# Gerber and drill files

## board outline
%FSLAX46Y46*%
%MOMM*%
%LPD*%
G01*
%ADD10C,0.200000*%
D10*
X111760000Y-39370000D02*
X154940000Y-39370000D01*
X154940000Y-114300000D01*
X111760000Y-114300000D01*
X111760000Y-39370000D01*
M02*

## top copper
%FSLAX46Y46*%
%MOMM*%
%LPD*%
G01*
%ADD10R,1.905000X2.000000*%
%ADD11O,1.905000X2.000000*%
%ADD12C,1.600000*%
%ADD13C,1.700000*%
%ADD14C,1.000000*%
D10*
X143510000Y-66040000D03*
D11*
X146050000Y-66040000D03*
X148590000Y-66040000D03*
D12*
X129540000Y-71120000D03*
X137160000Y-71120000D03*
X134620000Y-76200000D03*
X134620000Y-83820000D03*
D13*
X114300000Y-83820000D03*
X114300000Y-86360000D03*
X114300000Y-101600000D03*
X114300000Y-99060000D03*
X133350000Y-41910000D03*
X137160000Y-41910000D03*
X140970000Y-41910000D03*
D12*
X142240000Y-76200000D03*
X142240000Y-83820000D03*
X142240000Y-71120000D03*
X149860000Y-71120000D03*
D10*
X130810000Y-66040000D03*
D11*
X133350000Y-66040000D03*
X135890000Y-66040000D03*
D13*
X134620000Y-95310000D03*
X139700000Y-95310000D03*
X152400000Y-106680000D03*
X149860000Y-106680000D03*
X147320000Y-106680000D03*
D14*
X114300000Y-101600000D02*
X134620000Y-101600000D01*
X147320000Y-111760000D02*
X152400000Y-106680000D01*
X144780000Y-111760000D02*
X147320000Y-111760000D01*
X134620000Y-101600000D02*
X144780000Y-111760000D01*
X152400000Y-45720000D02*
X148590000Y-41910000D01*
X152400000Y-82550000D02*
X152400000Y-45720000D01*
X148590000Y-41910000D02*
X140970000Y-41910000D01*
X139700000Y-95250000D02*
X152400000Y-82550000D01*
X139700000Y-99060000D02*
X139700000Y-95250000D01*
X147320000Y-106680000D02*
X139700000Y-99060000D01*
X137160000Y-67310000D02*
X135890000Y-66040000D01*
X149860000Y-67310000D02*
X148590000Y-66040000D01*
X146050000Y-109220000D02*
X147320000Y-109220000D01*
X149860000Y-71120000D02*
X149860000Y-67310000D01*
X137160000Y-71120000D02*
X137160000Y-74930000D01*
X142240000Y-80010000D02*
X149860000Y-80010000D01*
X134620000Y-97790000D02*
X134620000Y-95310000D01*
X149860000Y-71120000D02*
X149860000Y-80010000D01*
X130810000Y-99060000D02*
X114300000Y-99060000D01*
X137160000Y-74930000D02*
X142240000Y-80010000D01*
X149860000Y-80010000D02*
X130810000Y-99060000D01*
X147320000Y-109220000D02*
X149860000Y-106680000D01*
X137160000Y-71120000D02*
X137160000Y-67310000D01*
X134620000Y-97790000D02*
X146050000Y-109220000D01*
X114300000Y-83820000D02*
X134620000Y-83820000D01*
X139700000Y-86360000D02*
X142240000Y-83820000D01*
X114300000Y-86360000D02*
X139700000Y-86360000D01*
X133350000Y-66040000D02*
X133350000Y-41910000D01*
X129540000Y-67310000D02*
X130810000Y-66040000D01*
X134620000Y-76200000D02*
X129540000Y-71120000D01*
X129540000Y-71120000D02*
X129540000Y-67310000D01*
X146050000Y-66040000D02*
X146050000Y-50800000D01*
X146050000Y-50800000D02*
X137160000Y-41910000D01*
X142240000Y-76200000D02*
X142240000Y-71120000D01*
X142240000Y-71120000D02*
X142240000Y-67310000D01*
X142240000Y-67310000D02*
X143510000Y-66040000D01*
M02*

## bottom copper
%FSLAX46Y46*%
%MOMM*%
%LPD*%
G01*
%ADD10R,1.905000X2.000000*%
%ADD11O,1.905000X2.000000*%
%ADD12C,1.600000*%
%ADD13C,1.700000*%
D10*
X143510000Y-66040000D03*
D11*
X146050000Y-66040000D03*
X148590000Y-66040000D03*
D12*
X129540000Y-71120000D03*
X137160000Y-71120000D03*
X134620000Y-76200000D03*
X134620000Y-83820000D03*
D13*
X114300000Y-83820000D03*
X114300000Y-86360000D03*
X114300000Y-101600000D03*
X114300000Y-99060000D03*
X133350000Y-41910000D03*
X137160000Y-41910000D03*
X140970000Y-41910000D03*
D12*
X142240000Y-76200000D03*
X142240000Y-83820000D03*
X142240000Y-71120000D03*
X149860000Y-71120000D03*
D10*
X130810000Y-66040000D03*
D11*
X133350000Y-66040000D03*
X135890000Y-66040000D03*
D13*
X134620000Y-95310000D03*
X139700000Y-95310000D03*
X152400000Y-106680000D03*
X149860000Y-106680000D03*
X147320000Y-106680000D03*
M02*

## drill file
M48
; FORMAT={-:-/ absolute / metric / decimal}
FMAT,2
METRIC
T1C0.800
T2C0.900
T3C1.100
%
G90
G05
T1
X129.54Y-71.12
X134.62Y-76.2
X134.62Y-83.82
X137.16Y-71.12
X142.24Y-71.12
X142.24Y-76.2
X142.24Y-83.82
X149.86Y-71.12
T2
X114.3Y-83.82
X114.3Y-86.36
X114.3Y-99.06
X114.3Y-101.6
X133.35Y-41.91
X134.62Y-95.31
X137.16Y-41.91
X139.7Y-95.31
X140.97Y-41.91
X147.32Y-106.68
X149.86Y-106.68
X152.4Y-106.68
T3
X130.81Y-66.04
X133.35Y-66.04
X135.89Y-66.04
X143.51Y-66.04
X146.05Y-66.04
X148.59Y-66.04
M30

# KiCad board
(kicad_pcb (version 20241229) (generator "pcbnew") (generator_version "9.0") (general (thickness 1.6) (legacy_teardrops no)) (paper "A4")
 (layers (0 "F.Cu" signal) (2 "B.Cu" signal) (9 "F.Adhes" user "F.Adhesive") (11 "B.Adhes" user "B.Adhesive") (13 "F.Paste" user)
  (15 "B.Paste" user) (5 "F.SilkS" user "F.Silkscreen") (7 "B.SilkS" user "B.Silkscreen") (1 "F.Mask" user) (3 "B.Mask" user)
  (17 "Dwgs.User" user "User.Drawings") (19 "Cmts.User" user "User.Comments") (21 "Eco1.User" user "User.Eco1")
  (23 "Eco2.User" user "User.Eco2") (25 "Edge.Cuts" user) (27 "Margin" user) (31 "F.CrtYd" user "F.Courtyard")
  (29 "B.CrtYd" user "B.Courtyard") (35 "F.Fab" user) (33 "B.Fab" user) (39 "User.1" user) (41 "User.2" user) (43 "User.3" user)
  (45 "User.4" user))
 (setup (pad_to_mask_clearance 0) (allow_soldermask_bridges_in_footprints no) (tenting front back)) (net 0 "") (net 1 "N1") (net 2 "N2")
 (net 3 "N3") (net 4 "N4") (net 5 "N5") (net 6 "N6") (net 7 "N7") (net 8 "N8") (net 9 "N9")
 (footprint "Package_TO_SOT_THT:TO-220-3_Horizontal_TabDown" (layer "F.Cu") (at 143.51 66.04)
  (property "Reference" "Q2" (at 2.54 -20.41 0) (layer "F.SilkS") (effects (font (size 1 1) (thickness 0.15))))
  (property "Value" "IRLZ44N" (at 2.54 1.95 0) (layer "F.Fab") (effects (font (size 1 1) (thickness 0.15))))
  (pad "1" thru_hole rect (at 0 0) (size 1.905 2) (drill 1.1) (layers "*.Cu" "*.Mask") (remove_unused_layers no) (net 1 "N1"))
  (pad "2" thru_hole oval (at 2.54 0) (size 1.905 2) (drill 1.1) (layers "*.Cu" "*.Mask") (remove_unused_layers no) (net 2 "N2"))
  (pad "3" thru_hole oval (at 5.08 0) (size 1.905 2) (drill 1.1) (layers "*.Cu" "*.Mask") (remove_unused_layers no) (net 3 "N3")))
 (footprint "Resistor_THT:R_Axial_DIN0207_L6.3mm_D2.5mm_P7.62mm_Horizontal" (layer "F.Cu") (at 129.54 71.12)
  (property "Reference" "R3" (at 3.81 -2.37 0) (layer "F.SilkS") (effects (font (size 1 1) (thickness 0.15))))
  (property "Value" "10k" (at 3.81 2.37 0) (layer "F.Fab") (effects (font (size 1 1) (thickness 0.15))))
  (pad "1" thru_hole circle (at 0 0) (size 1.6 1.6) (drill 0.8) (layers "*.Cu" "*.Mask") (remove_unused_layers no) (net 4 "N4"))
  (pad "2" thru_hole circle (at 7.62 0) (size 1.6 1.6) (drill 0.8) (layers "*.Cu" "*.Mask") (remove_unused_layers no) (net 3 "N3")))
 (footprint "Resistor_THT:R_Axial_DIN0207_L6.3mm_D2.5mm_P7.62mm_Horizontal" (layer "F.Cu") (at 134.62 76.2 -90)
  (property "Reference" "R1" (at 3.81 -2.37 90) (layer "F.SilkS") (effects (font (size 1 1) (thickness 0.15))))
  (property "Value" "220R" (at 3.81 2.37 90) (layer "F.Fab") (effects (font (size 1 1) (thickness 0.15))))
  (pad "1" thru_hole circle (at 0 0 270) (size 1.6 1.6) (drill 0.8) (layers "*.Cu" "*.Mask") (remove_unused_layers no) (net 4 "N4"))
  (pad "2" thru_hole circle (at 7.62 0 270) (size 1.6 1.6) (drill 0.8) (layers "*.Cu" "*.Mask") (remove_unused_layers no) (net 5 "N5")))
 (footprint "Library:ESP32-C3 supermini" (layer "F.Cu") (at 121.92 91.44)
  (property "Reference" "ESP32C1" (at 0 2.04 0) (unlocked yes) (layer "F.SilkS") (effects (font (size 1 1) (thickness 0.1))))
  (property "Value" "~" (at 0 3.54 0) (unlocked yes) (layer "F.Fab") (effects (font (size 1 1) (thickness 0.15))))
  (pad "0" thru_hole circle (at -7.62 -7.62) (size 1.7 1.7) (drill 0.9) (layers "*.Cu" "*.Mask") (remove_unused_layers yes)
   (keep_end_layers yes) (zone_layer_connections) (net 5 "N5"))
  (pad "1" thru_hole circle (at -7.62 -5.08) (size 1.7 1.7) (drill 0.9) (layers "*.Cu" "*.Mask") (remove_unused_layers yes)
   (keep_end_layers yes) (zone_layer_connections) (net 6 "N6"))
  (pad "5V" thru_hole circle (at -7.62 10.16) (size 1.7 1.7) (drill 0.9) (layers "*.Cu" "*.Mask") (remove_unused_layers yes)
   (keep_end_layers yes) (zone_layer_connections) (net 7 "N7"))
  (pad "GND" thru_hole circle (at -7.62 7.62) (size 1.7 1.7) (drill 0.9) (layers "*.Cu" "*.Mask") (remove_unused_layers yes)
   (keep_end_layers yes) (zone_layer_connections) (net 3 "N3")))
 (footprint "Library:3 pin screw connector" (layer "F.Cu") (at 137.16 41.91)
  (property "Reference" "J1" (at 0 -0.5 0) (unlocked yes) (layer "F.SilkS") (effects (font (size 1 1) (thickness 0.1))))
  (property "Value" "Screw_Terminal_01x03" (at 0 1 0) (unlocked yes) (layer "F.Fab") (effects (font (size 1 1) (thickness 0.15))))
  (pad "1" thru_hole circle (at -3.81 0) (size 1.7 1.7) (drill 0.9) (layers "*.Cu" "*.Mask") (remove_unused_layers yes)
   (keep_end_layers yes) (zone_layer_connections) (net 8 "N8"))
  (pad "2" thru_hole circle (at 0 0) (size 1.7 1.7) (drill 0.9) (layers "*.Cu" "*.Mask") (remove_unused_layers yes) (keep_end_layers yes)
   (zone_layer_connections) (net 2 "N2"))
  (pad "3" thru_hole circle (at 3.81 0) (size 1.7 1.7) (drill 0.9) (layers "*.Cu" "*.Mask") (remove_unused_layers yes) (keep_end_layers yes)
   (zone_layer_connections) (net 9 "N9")))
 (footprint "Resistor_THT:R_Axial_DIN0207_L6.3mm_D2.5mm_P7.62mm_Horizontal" (layer "F.Cu") (at 142.24 76.2 -90)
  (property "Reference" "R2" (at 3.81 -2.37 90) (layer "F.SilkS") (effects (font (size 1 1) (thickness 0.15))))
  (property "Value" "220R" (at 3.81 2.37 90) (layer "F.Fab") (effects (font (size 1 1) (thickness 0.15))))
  (pad "1" thru_hole circle (at 0 0 270) (size 1.6 1.6) (drill 0.8) (layers "*.Cu" "*.Mask") (remove_unused_layers no) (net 1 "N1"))
  (pad "2" thru_hole circle (at 7.62 0 270) (size 1.6 1.6) (drill 0.8) (layers "*.Cu" "*.Mask") (remove_unused_layers no) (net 6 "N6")))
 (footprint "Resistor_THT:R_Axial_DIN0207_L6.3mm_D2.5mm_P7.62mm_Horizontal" (layer "F.Cu") (at 142.24 71.12)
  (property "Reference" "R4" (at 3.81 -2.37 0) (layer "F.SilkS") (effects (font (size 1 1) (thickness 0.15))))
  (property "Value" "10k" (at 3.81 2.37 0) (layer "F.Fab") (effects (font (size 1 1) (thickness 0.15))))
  (pad "1" thru_hole circle (at 0 0) (size 1.6 1.6) (drill 0.8) (layers "*.Cu" "*.Mask") (remove_unused_layers no) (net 1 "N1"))
  (pad "2" thru_hole circle (at 7.62 0) (size 1.6 1.6) (drill 0.8) (layers "*.Cu" "*.Mask") (remove_unused_layers no) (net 3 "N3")))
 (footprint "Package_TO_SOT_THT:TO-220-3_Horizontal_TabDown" (layer "F.Cu") (at 130.81 66.04)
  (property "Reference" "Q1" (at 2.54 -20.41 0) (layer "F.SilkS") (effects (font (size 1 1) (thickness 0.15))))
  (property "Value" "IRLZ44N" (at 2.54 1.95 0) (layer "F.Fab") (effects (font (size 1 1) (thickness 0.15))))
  (pad "1" thru_hole rect (at 0 0) (size 1.905 2) (drill 1.1) (layers "*.Cu" "*.Mask") (remove_unused_layers no) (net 4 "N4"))
  (pad "2" thru_hole oval (at 2.54 0) (size 1.905 2) (drill 1.1) (layers "*.Cu" "*.Mask") (remove_unused_layers no) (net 8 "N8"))
  (pad "3" thru_hole oval (at 5.08 0) (size 1.905 2) (drill 1.1) (layers "*.Cu" "*.Mask") (remove_unused_layers no) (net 3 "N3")))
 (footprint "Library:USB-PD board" (layer "F.Cu") (at 137.16 97.85)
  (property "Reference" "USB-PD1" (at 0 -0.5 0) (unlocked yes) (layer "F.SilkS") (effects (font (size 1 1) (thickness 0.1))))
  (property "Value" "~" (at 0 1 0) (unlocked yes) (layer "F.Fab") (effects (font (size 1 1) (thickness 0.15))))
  (pad "GND" thru_hole circle (at -2.54 -2.54) (size 1.7 1.7) (drill 0.9) (layers "*.Cu" "*.Mask") (remove_unused_layers yes)
   (keep_end_layers yes) (zone_layer_connections) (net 3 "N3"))
  (pad "VBUS" thru_hole circle (at 2.54 -2.54) (size 1.7 1.7) (drill 0.9) (layers "*.Cu" "*.Mask") (remove_unused_layers yes)
   (keep_end_layers yes) (zone_layer_connections) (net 9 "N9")))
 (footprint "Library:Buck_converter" (layer "F.Cu") (at 148.59 111.76 180)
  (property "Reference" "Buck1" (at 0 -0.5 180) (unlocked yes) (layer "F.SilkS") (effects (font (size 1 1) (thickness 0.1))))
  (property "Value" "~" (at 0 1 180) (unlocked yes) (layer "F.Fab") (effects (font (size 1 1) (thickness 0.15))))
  (pad "1" thru_hole circle (at -3.81 5.08 180) (size 1.7 1.7) (drill 0.9) (layers "*.Cu" "*.Mask") (remove_unused_layers yes)
   (keep_end_layers yes) (zone_layer_connections) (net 7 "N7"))
  (pad "2" thru_hole circle (at -1.27 5.08 180) (size 1.7 1.7) (drill 0.9) (layers "*.Cu" "*.Mask") (remove_unused_layers yes)
   (keep_end_layers yes) (zone_layer_connections) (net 3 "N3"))
  (pad "3" thru_hole circle (at 1.27 5.08 180) (size 1.7 1.7) (drill 0.9) (layers "*.Cu" "*.Mask") (remove_unused_layers yes)
   (keep_end_layers yes) (zone_layer_connections) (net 9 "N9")))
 (gr_rect (start 111.76 39.37) (end 154.94 114.3) (stroke (width 0.2) (type solid)) (fill no) (layer "Edge.Cuts"))
 (segment (start 114.3 101.6) (end 134.62 101.6) (width 1) (layer "F.Cu") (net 7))
 (segment (start 147.32 111.76) (end 152.4 106.68) (width 1) (layer "F.Cu") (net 7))
 (segment (start 144.78 111.76) (end 147.32 111.76) (width 1) (layer "F.Cu") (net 7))
 (segment (start 134.62 101.6) (end 144.78 111.76) (width 1) (layer "F.Cu") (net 7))
 (segment (start 152.4 45.72) (end 148.59 41.91) (width 1) (layer "F.Cu") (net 9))
 (segment (start 152.4 82.55) (end 152.4 45.72) (width 1) (layer "F.Cu") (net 9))
 (segment (start 148.59 41.91) (end 140.97 41.91) (width 1) (layer "F.Cu") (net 9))
 (segment (start 139.7 95.25) (end 152.4 82.55) (width 1) (layer "F.Cu") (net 9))
 (segment (start 139.7 99.06) (end 139.7 95.25) (width 1) (layer "F.Cu") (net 9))
 (segment (start 147.32 106.68) (end 139.7 99.06) (width 1) (layer "F.Cu") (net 9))
 (segment (start 137.16 67.31) (end 135.89 66.04) (width 1) (layer "F.Cu") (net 3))
 (segment (start 149.86 67.31) (end 148.59 66.04) (width 1) (layer "F.Cu") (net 3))
 (segment (start 146.05 109.22) (end 147.32 109.22) (width 1) (layer "F.Cu") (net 3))
 (segment (start 149.86 71.12) (end 149.86 67.31) (width 1) (layer "F.Cu") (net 3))
 (segment (start 137.16 71.12) (end 137.16 74.93) (width 1) (layer "F.Cu") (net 3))
 (segment (start 142.24 80.01) (end 149.86 80.01) (width 1) (layer "F.Cu") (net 3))
 (segment (start 134.62 97.79) (end 134.62 95.31) (width 1) (layer "F.Cu") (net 3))
 (segment (start 149.86 71.12) (end 149.86 80.01) (width 1) (layer "F.Cu") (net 3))
 (segment (start 130.81 99.06) (end 114.3 99.06) (width 1) (layer "F.Cu") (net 3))
 (segment (start 137.16 74.93) (end 142.24 80.01) (width 1) (layer "F.Cu") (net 3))
 (segment (start 149.86 80.01) (end 130.81 99.06) (width 1) (layer "F.Cu") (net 3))
 (segment (start 147.32 109.22) (end 149.86 106.68) (width 1) (layer "F.Cu") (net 3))
 (segment (start 137.16 71.12) (end 137.16 67.31) (width 1) (layer "F.Cu") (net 3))
 (segment (start 134.62 97.79) (end 146.05 109.22) (width 1) (layer "F.Cu") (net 3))
 (segment (start 114.3 83.82) (end 134.62 83.82) (width 1) (layer "F.Cu") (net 5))
 (segment (start 139.7 86.36) (end 142.24 83.82) (width 1) (layer "F.Cu") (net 6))
 (segment (start 114.3 86.36) (end 139.7 86.36) (width 1) (layer "F.Cu") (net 6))
 (segment (start 133.35 66.04) (end 133.35 41.91) (width 1) (layer "F.Cu") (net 8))
 (segment (start 129.54 67.31) (end 130.81 66.04) (width 1) (layer "F.Cu") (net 4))
 (segment (start 134.62 76.2) (end 129.54 71.12) (width 1) (layer "F.Cu") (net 4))
 (segment (start 129.54 71.12) (end 129.54 67.31) (width 1) (layer "F.Cu") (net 4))
 (segment (start 146.05 66.04) (end 146.05 50.8) (width 1) (layer "F.Cu") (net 2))
 (segment (start 146.05 50.8) (end 137.16 41.91) (width 1) (layer "F.Cu") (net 2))
 (segment (start 142.24 76.2) (end 142.24 71.12) (width 1) (layer "F.Cu") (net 1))
 (segment (start 142.24 71.12) (end 142.24 67.31) (width 1) (layer "F.Cu") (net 1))
 (segment (start 142.24 67.31) (end 143.51 66.04) (width 1) (layer "F.Cu") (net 1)))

